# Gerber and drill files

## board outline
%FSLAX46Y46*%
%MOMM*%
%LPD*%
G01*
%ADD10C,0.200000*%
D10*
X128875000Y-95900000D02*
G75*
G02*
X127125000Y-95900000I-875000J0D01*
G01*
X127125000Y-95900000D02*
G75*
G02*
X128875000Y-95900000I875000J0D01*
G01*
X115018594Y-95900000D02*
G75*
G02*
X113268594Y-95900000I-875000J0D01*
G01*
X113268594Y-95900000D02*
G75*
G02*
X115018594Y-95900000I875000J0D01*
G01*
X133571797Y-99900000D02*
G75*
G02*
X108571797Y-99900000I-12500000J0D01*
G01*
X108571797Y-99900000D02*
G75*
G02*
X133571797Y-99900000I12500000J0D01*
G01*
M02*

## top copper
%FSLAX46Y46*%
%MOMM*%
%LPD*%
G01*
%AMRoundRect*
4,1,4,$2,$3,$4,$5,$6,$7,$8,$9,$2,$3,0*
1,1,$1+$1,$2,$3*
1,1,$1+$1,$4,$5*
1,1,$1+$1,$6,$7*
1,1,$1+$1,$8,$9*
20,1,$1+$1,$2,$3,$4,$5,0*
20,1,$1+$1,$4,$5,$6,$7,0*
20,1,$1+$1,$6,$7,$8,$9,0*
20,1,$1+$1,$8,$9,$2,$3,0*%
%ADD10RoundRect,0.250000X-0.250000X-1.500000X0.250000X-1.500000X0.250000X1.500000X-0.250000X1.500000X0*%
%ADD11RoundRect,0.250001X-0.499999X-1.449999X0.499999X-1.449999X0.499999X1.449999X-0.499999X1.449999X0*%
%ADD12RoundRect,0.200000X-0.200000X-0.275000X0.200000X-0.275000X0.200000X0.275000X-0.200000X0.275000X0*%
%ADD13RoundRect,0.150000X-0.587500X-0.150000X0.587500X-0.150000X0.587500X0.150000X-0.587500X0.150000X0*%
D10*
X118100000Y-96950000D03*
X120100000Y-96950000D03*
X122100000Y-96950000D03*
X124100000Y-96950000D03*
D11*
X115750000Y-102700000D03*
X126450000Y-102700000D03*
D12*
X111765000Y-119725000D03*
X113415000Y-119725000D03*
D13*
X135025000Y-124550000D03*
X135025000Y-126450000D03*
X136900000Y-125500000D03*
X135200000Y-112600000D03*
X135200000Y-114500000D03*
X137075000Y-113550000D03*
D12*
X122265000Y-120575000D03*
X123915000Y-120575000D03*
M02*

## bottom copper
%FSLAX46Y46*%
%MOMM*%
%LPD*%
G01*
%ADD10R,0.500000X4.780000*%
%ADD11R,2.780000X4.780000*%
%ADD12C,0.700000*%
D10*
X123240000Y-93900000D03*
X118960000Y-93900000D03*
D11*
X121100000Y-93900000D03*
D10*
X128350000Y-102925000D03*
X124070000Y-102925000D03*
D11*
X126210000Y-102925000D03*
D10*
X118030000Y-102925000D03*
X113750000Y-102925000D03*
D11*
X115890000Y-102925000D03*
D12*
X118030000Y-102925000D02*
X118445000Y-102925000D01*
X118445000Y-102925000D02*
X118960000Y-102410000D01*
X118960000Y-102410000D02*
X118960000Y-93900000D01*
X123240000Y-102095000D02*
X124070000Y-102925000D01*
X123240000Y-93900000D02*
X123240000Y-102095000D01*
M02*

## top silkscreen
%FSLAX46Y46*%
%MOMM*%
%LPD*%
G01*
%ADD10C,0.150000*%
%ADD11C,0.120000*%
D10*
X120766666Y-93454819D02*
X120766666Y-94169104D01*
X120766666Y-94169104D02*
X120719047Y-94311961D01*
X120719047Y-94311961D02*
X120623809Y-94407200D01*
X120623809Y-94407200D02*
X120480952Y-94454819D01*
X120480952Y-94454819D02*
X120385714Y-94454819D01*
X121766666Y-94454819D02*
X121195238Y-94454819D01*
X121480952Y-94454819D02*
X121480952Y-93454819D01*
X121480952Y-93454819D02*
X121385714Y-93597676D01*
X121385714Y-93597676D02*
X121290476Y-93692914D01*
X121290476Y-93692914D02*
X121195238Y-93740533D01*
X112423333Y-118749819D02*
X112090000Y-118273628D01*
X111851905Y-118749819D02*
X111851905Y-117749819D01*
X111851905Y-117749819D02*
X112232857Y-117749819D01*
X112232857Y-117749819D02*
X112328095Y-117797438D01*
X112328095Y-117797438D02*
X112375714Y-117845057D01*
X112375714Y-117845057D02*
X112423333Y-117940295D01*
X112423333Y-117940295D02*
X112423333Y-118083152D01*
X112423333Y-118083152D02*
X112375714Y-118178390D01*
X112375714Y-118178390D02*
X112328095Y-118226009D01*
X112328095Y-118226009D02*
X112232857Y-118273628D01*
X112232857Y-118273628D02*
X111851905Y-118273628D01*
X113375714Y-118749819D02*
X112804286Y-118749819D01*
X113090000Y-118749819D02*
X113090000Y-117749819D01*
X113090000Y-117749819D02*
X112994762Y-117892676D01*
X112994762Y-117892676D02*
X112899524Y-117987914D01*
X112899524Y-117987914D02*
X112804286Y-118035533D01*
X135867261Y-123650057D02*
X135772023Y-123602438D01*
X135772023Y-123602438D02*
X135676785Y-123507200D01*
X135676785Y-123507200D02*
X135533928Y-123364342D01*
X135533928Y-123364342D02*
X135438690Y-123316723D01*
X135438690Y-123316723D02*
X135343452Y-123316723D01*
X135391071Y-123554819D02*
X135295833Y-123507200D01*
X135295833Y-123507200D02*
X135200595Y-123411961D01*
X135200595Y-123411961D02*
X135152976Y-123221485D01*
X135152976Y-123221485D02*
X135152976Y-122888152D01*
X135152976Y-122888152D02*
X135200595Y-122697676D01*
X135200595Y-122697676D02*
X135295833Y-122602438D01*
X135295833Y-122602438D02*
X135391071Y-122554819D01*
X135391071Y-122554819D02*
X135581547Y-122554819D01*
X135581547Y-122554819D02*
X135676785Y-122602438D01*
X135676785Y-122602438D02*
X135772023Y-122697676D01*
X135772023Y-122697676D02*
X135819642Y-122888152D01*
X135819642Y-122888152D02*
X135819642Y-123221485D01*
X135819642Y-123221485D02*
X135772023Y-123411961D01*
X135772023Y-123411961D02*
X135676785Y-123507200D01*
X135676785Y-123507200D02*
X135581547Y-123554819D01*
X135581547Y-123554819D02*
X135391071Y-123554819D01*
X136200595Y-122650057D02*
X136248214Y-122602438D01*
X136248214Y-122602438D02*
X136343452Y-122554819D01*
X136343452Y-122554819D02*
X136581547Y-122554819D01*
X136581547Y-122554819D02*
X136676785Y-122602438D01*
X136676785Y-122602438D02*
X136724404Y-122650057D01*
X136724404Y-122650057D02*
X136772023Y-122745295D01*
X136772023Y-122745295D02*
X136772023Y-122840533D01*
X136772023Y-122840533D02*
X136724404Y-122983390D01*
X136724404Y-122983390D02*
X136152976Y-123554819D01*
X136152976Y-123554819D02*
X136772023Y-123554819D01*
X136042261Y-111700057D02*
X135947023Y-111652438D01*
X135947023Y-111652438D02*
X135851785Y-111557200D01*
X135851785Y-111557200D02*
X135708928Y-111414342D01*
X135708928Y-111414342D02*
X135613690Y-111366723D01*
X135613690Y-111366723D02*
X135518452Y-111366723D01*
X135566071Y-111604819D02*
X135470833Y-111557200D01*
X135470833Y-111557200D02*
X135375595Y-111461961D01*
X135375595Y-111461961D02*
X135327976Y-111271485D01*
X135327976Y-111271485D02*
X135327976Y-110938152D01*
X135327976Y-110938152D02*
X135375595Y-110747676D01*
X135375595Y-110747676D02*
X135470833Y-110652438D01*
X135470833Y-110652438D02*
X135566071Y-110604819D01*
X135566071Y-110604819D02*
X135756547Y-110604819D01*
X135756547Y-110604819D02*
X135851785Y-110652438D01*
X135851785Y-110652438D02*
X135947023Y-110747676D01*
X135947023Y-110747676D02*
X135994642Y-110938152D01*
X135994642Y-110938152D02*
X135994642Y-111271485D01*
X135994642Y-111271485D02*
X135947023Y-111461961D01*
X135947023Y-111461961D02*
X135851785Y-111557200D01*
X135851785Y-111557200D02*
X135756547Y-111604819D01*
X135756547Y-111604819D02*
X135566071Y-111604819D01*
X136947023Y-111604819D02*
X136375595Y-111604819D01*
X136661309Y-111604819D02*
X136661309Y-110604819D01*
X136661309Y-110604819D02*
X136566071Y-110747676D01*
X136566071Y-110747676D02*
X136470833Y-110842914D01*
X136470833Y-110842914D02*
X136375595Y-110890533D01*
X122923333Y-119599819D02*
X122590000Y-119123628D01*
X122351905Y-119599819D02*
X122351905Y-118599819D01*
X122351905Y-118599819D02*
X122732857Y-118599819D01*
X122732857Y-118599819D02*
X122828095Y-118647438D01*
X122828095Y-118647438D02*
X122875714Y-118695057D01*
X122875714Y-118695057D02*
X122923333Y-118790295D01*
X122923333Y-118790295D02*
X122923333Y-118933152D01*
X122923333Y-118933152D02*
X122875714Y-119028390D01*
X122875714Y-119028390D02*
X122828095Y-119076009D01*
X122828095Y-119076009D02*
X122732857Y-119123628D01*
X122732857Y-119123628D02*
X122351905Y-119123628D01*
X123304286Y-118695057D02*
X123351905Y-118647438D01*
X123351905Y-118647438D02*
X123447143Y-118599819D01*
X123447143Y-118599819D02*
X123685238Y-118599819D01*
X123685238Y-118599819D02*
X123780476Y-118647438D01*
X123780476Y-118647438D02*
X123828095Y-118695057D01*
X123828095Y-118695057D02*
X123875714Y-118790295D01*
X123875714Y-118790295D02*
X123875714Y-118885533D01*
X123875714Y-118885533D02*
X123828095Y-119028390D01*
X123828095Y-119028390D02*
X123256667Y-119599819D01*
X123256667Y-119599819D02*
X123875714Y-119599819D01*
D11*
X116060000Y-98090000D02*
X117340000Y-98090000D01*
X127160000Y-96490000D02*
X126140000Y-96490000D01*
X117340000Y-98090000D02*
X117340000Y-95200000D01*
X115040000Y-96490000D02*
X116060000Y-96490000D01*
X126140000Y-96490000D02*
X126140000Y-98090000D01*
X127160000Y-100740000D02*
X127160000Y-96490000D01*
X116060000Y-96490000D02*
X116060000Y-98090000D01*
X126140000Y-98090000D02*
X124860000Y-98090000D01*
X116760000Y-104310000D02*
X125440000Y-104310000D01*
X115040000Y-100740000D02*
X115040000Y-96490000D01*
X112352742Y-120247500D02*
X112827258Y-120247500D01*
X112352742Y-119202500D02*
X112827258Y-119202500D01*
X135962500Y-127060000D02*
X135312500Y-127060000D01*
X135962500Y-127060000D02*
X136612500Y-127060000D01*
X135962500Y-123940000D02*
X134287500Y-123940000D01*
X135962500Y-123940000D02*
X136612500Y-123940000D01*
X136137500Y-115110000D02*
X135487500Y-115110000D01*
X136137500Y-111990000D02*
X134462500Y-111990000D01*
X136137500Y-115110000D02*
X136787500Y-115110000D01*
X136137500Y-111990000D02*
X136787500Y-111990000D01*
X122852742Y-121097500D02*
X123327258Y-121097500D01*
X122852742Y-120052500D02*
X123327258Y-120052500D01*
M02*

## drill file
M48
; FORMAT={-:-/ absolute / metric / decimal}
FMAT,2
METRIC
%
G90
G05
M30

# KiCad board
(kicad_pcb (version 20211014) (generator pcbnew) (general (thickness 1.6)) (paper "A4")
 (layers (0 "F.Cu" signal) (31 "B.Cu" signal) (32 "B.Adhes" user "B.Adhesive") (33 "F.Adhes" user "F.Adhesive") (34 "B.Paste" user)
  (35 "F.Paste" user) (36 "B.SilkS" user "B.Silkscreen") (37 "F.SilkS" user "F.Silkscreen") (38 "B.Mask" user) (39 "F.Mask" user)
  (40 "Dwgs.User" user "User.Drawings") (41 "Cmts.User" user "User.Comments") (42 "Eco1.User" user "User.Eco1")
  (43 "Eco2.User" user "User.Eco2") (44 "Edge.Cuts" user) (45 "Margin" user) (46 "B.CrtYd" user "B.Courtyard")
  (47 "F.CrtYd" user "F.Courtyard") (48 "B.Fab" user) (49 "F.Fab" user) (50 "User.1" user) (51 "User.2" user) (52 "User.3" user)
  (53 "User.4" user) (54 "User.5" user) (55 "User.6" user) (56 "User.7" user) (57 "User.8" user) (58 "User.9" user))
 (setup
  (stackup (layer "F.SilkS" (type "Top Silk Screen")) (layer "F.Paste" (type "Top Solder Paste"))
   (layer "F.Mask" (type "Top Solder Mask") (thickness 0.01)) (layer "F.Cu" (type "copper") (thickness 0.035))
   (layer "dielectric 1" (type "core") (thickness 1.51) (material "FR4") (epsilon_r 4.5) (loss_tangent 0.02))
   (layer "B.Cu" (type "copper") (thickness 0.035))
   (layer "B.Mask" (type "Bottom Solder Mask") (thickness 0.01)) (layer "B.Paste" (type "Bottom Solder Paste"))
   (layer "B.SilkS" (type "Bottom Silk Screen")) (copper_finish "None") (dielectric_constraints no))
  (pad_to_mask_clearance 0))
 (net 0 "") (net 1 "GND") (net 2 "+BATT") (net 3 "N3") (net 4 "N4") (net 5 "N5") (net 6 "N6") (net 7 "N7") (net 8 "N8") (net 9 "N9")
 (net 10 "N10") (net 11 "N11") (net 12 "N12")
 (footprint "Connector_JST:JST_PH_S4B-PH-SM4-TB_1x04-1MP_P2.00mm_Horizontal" (layer "F.Cu") (at 121.1 99.8)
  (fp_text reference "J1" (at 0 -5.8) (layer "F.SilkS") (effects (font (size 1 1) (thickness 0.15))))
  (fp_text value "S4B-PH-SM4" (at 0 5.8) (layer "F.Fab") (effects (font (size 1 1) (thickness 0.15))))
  (fp_line (start -5.04 -1.71) (end -3.76 -1.71) (layer "F.SilkS") (width 0.12))
  (fp_line (start 6.06 -3.31) (end 5.04 -3.31) (layer "F.SilkS") (width 0.12))
  (fp_line (start -3.76 -1.71) (end -3.76 -4.6) (layer "F.SilkS") (width 0.12))
  (fp_line (start -6.06 -3.31) (end -5.04 -3.31) (layer "F.SilkS") (width 0.12))
  (fp_line (start 5.04 -3.31) (end 5.04 -1.71) (layer "F.SilkS") (width 0.12))
  (fp_line (start 6.06 0.94) (end 6.06 -3.31) (layer "F.SilkS") (width 0.12))
  (fp_line (start -5.04 -3.31) (end -5.04 -1.71) (layer "F.SilkS") (width 0.12))
  (fp_line (start 5.04 -1.71) (end 3.76 -1.71) (layer "F.SilkS") (width 0.12))
  (fp_line (start -4.34 4.51) (end 4.34 4.51) (layer "F.SilkS") (width 0.12))
  (fp_line (start -6.06 0.94) (end -6.06 -3.31) (layer "F.SilkS") (width 0.12))
  (pad "1" smd roundrect (at -3 -2.85) (size 1 3.5) (layers "F.Cu" "F.Paste" "F.Mask") (roundrect_rratio 0.25) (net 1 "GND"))
  (pad "2" smd roundrect (at -1 -2.85) (size 1 3.5) (layers "F.Cu" "F.Paste" "F.Mask") (roundrect_rratio 0.25) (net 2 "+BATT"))
  (pad "3" smd roundrect (at 1 -2.85) (size 1 3.5) (layers "F.Cu" "F.Paste" "F.Mask") (roundrect_rratio 0.25) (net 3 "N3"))
  (pad "4" smd roundrect (at 3 -2.85) (size 1 3.5) (layers "F.Cu" "F.Paste" "F.Mask") (roundrect_rratio 0.25) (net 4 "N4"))
  (pad "MP" smd roundrect (at -5.35 2.9) (size 1.5 3.4) (layers "F.Cu" "F.Paste" "F.Mask") (roundrect_rratio 0.166667))
  (pad "MP" smd roundrect (at 5.35 2.9) (size 1.5 3.4) (layers "F.Cu" "F.Paste" "F.Mask") (roundrect_rratio 0.166667)))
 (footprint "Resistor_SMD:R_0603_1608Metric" (layer "F.Cu") (at 112.59 119.725)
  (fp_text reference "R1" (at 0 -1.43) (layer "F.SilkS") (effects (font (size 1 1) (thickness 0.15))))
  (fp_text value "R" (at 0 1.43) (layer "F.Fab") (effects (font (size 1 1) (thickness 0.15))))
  (fp_line (start -0.237258 0.5225) (end 0.237258 0.5225) (layer "F.SilkS") (width 0.12))
  (fp_line (start -0.237258 -0.5225) (end 0.237258 -0.5225) (layer "F.SilkS") (width 0.12))
  (pad "1" smd roundrect (at -0.825 0) (size 0.8 0.95) (layers "F.Cu" "F.Paste" "F.Mask") (roundrect_rratio 0.25) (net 2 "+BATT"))
  (pad "2" smd roundrect (at 0.825 0) (size 0.8 0.95) (layers "F.Cu" "F.Paste" "F.Mask") (roundrect_rratio 0.25) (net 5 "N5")))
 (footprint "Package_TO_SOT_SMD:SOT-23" (layer "F.Cu") (at 135.9625 125.5)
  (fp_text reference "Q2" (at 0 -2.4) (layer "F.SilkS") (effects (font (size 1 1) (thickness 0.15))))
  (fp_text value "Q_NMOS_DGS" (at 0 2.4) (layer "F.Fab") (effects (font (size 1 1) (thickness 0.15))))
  (fp_line (start 0 1.56) (end -0.65 1.56) (layer "F.SilkS") (width 0.12))
  (fp_line (start 0 1.56) (end 0.65 1.56) (layer "F.SilkS") (width 0.12))
  (fp_line (start 0 -1.56) (end -1.675 -1.56) (layer "F.SilkS") (width 0.12))
  (fp_line (start 0 -1.56) (end 0.65 -1.56) (layer "F.SilkS") (width 0.12))
  (pad "1" smd roundrect (at -0.9375 -0.95) (size 1.475 0.6) (layers "F.Cu" "F.Paste" "F.Mask") (roundrect_rratio 0.25) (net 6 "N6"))
  (pad "2" smd roundrect (at -0.9375 0.95) (size 1.475 0.6) (layers "F.Cu" "F.Paste" "F.Mask") (roundrect_rratio 0.25) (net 5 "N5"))
  (pad "3" smd roundrect (at 0.9375 0) (size 1.475 0.6) (layers "F.Cu" "F.Paste" "F.Mask") (roundrect_rratio 0.25) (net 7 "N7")))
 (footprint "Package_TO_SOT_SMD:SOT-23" (layer "F.Cu") (at 136.1375 113.55)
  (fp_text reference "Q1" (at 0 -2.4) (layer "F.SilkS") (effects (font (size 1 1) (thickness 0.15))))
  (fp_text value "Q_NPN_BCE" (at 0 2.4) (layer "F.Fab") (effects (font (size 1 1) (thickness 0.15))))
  (fp_line (start 0 1.56) (end -0.65 1.56) (layer "F.SilkS") (width 0.12))
  (fp_line (start 0 -1.56) (end -1.675 -1.56) (layer "F.SilkS") (width 0.12))
  (fp_line (start 0 1.56) (end 0.65 1.56) (layer "F.SilkS") (width 0.12))
  (fp_line (start 0 -1.56) (end 0.65 -1.56) (layer "F.SilkS") (width 0.12))
  (pad "1" smd roundrect (at -0.9375 -0.95) (size 1.475 0.6) (layers "F.Cu" "F.Paste" "F.Mask") (roundrect_rratio 0.25) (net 7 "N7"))
  (pad "2" smd roundrect (at -0.9375 0.95) (size 1.475 0.6) (layers "F.Cu" "F.Paste" "F.Mask") (roundrect_rratio 0.25) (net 5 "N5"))
  (pad "3" smd roundrect (at 0.9375 0) (size 1.475 0.6) (layers "F.Cu" "F.Paste" "F.Mask") (roundrect_rratio 0.25) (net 1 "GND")))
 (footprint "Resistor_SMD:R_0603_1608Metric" (layer "F.Cu") (at 123.09 120.575)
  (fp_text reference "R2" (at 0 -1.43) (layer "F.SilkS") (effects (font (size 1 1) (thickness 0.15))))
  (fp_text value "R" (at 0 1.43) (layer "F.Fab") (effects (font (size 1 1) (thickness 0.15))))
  (fp_line (start -0.237258 0.5225) (end 0.237258 0.5225) (layer "F.SilkS") (width 0.12))
  (fp_line (start -0.237258 -0.5225) (end 0.237258 -0.5225) (layer "F.SilkS") (width 0.12))
  (pad "1" smd roundrect (at -0.825 0) (size 0.8 0.95) (layers "F.Cu" "F.Paste" "F.Mask") (roundrect_rratio 0.25) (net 7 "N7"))
  (pad "2" smd roundrect (at 0.825 0) (size 0.8 0.95) (layers "F.Cu" "F.Paste" "F.Mask") (roundrect_rratio 0.25) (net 1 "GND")))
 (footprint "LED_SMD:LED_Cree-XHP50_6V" (layer "B.Cu") (at 121.1 93.9 180)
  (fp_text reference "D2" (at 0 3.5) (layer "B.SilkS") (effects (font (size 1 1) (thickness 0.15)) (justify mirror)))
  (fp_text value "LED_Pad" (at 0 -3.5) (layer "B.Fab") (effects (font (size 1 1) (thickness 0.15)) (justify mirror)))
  (pad "" smd rect (at -0.61 0.525 180) (size 0.97 0.8) (layers "B.Paste"))
  (pad "" smd rect (at -0.61 -0.525 180) (size 0.97 0.8) (layers "B.Paste"))
  (pad "" smd rect (at 2.14 -1.32 180) (size 0.5 2.14) (layers "B.Paste"))
  (pad "" smd rect (at -0.61 1.575 180) (size 0.97 0.8) (layers "B.Paste"))
  (pad "" smd rect (at 0.61 -1.575 180) (size 0.97 0.8) (layers "B.Paste"))
  (pad "" smd rect (at 0.61 1.575 180) (size 0.97 0.8) (layers "B.Paste"))
  (pad "" smd rect (at 0.61 -0.525 180) (size 0.97 0.8) (layers "B.Paste"))
  (pad "" smd rect (at 0.61 0.525 180) (size 0.97 0.8) (layers "B.Paste"))
  (pad "" smd rect (at -2.14 1.32 180) (size 0.5 2.14) (layers "B.Paste"))
  (pad "" smd rect (at -0.61 -1.575 180) (size 0.97 0.8) (layers "B.Paste"))
  (pad "" smd rect (at -2.14 -1.32 180) (size 0.5 2.14) (layers "B.Paste"))
  (pad "" smd rect (at 2.14 1.32 180) (size 0.5 2.14) (layers "B.Paste"))
  (pad "1" smd rect (at -2.14 0 180) (size 0.5 4.78) (layers "B.Cu" "B.Mask") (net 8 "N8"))
  (pad "2" smd rect (at 2.14 0 180) (size 0.5 4.78) (layers "B.Cu" "B.Mask") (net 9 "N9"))
  (pad "3" smd rect (at 0 0 180) (size 2.78 4.78) (layers "B.Cu" "B.Mask") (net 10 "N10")))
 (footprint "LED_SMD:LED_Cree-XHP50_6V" (layer "B.Cu") (at 126.21 102.925 180)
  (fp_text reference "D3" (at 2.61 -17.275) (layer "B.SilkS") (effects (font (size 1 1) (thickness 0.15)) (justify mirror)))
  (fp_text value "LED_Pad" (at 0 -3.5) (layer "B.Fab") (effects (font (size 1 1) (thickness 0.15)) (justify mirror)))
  (pad "" smd rect (at -0.61 -1.575 180) (size 0.97 0.8) (layers "B.Paste"))
  (pad "" smd rect (at 2.14 1.32 180) (size 0.5 2.14) (layers "B.Paste"))
  (pad "" smd rect (at 0.61 1.575 180) (size 0.97 0.8) (layers "B.Paste"))
  (pad "" smd rect (at 0.61 -1.575 180) (size 0.97 0.8) (layers "B.Paste"))
  (pad "" smd rect (at 2.14 -1.32 180) (size 0.5 2.14) (layers "B.Paste"))
  (pad "" smd rect (at -0.61 0.525 180) (size 0.97 0.8) (layers "B.Paste"))
  (pad "" smd rect (at 0.61 -0.525 180) (size 0.97 0.8) (layers "B.Paste"))
  (pad "" smd rect (at -2.14 1.32 180) (size 0.5 2.14) (layers "B.Paste"))
  (pad "" smd rect (at -0.61 -0.525 180) (size 0.97 0.8) (layers "B.Paste"))
  (pad "" smd rect (at 0.61 0.525 180) (size 0.97 0.8) (layers "B.Paste"))
  (pad "" smd rect (at -2.14 -1.32 180) (size 0.5 2.14) (layers "B.Paste"))
  (pad "" smd rect (at -0.61 1.575 180) (size 0.97 0.8) (layers "B.Paste"))
  (pad "1" smd rect (at -2.14 0 180) (size 0.5 4.78) (layers "B.Cu" "B.Mask") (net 6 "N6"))
  (pad "2" smd rect (at 2.14 0 180) (size 0.5 4.78) (layers "B.Cu" "B.Mask") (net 8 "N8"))
  (pad "3" smd rect (at 0 0 180) (size 2.78 4.78) (layers "B.Cu" "B.Mask") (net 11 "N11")))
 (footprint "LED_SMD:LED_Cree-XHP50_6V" (layer "B.Cu") (at 115.89 102.925 180)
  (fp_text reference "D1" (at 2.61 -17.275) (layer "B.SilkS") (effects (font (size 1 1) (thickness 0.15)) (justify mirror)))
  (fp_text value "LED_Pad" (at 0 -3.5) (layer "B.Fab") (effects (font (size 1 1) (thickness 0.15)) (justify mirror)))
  (pad "" smd rect (at -0.61 0.525 180) (size 0.97 0.8) (layers "B.Paste"))
  (pad "" smd rect (at -2.14 -1.32 180) (size 0.5 2.14) (layers "B.Paste"))
  (pad "" smd rect (at 0.61 -0.525 180) (size 0.97 0.8) (layers "B.Paste"))
  (pad "" smd rect (at -0.61 -1.575 180) (size 0.97 0.8) (layers "B.Paste"))
  (pad "" smd rect (at -0.61 1.575 180) (size 0.97 0.8) (layers "B.Paste"))
  (pad "" smd rect (at -2.14 1.32 180) (size 0.5 2.14) (layers "B.Paste"))
  (pad "" smd rect (at 0.61 -1.575 180) (size 0.97 0.8) (layers "B.Paste"))
  (pad "" smd rect (at -0.61 -0.525 180) (size 0.97 0.8) (layers "B.Paste"))
  (pad "" smd rect (at 0.61 0.525 180) (size 0.97 0.8) (layers "B.Paste"))
  (pad "" smd rect (at 2.14 1.32 180) (size 0.5 2.14) (layers "B.Paste"))
  (pad "" smd rect (at 0.61 1.575 180) (size 0.97 0.8) (layers "B.Paste"))
  (pad "" smd rect (at 2.14 -1.32 180) (size 0.5 2.14) (layers "B.Paste"))
  (pad "1" smd rect (at -2.14 0 180) (size 0.5 4.78) (layers "B.Cu" "B.Mask") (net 9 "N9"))
  (pad "2" smd rect (at 2.14 0 180) (size 0.5 4.78) (layers "B.Cu" "B.Mask") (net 2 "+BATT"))
  (pad "3" smd rect (at 0 0 180) (size 2.78 4.78) (layers "B.Cu" "B.Mask") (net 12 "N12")))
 (gr_circle (center 128 95.9) (end 128.875 95.9) (layer "Edge.Cuts") (width 0.2) (fill none))
 (gr_circle (center 114.143594 95.9) (end 115.018594 95.9) (layer "Edge.Cuts") (width 0.2) (fill none))
 (gr_circle (center 121.071797 99.9) (end 133.571797 99.9) (layer "Edge.Cuts") (width 0.2) (fill none))
 (segment (start 118.03 102.925) (end 118.445 102.925) (width 0.7) (layer "B.Cu") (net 9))
 (segment (start 118.445 102.925) (end 118.96 102.41) (width 0.7) (layer "B.Cu") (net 9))
 (segment (start 118.96 102.41) (end 118.96 93.9) (width 0.7) (layer "B.Cu") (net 9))
 (segment (start 123.24 102.095) (end 124.07 102.925) (width 0.7) (layer "B.Cu") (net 8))
 (segment (start 123.24 93.9) (end 123.24 102.095) (width 0.7) (layer "B.Cu") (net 8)))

